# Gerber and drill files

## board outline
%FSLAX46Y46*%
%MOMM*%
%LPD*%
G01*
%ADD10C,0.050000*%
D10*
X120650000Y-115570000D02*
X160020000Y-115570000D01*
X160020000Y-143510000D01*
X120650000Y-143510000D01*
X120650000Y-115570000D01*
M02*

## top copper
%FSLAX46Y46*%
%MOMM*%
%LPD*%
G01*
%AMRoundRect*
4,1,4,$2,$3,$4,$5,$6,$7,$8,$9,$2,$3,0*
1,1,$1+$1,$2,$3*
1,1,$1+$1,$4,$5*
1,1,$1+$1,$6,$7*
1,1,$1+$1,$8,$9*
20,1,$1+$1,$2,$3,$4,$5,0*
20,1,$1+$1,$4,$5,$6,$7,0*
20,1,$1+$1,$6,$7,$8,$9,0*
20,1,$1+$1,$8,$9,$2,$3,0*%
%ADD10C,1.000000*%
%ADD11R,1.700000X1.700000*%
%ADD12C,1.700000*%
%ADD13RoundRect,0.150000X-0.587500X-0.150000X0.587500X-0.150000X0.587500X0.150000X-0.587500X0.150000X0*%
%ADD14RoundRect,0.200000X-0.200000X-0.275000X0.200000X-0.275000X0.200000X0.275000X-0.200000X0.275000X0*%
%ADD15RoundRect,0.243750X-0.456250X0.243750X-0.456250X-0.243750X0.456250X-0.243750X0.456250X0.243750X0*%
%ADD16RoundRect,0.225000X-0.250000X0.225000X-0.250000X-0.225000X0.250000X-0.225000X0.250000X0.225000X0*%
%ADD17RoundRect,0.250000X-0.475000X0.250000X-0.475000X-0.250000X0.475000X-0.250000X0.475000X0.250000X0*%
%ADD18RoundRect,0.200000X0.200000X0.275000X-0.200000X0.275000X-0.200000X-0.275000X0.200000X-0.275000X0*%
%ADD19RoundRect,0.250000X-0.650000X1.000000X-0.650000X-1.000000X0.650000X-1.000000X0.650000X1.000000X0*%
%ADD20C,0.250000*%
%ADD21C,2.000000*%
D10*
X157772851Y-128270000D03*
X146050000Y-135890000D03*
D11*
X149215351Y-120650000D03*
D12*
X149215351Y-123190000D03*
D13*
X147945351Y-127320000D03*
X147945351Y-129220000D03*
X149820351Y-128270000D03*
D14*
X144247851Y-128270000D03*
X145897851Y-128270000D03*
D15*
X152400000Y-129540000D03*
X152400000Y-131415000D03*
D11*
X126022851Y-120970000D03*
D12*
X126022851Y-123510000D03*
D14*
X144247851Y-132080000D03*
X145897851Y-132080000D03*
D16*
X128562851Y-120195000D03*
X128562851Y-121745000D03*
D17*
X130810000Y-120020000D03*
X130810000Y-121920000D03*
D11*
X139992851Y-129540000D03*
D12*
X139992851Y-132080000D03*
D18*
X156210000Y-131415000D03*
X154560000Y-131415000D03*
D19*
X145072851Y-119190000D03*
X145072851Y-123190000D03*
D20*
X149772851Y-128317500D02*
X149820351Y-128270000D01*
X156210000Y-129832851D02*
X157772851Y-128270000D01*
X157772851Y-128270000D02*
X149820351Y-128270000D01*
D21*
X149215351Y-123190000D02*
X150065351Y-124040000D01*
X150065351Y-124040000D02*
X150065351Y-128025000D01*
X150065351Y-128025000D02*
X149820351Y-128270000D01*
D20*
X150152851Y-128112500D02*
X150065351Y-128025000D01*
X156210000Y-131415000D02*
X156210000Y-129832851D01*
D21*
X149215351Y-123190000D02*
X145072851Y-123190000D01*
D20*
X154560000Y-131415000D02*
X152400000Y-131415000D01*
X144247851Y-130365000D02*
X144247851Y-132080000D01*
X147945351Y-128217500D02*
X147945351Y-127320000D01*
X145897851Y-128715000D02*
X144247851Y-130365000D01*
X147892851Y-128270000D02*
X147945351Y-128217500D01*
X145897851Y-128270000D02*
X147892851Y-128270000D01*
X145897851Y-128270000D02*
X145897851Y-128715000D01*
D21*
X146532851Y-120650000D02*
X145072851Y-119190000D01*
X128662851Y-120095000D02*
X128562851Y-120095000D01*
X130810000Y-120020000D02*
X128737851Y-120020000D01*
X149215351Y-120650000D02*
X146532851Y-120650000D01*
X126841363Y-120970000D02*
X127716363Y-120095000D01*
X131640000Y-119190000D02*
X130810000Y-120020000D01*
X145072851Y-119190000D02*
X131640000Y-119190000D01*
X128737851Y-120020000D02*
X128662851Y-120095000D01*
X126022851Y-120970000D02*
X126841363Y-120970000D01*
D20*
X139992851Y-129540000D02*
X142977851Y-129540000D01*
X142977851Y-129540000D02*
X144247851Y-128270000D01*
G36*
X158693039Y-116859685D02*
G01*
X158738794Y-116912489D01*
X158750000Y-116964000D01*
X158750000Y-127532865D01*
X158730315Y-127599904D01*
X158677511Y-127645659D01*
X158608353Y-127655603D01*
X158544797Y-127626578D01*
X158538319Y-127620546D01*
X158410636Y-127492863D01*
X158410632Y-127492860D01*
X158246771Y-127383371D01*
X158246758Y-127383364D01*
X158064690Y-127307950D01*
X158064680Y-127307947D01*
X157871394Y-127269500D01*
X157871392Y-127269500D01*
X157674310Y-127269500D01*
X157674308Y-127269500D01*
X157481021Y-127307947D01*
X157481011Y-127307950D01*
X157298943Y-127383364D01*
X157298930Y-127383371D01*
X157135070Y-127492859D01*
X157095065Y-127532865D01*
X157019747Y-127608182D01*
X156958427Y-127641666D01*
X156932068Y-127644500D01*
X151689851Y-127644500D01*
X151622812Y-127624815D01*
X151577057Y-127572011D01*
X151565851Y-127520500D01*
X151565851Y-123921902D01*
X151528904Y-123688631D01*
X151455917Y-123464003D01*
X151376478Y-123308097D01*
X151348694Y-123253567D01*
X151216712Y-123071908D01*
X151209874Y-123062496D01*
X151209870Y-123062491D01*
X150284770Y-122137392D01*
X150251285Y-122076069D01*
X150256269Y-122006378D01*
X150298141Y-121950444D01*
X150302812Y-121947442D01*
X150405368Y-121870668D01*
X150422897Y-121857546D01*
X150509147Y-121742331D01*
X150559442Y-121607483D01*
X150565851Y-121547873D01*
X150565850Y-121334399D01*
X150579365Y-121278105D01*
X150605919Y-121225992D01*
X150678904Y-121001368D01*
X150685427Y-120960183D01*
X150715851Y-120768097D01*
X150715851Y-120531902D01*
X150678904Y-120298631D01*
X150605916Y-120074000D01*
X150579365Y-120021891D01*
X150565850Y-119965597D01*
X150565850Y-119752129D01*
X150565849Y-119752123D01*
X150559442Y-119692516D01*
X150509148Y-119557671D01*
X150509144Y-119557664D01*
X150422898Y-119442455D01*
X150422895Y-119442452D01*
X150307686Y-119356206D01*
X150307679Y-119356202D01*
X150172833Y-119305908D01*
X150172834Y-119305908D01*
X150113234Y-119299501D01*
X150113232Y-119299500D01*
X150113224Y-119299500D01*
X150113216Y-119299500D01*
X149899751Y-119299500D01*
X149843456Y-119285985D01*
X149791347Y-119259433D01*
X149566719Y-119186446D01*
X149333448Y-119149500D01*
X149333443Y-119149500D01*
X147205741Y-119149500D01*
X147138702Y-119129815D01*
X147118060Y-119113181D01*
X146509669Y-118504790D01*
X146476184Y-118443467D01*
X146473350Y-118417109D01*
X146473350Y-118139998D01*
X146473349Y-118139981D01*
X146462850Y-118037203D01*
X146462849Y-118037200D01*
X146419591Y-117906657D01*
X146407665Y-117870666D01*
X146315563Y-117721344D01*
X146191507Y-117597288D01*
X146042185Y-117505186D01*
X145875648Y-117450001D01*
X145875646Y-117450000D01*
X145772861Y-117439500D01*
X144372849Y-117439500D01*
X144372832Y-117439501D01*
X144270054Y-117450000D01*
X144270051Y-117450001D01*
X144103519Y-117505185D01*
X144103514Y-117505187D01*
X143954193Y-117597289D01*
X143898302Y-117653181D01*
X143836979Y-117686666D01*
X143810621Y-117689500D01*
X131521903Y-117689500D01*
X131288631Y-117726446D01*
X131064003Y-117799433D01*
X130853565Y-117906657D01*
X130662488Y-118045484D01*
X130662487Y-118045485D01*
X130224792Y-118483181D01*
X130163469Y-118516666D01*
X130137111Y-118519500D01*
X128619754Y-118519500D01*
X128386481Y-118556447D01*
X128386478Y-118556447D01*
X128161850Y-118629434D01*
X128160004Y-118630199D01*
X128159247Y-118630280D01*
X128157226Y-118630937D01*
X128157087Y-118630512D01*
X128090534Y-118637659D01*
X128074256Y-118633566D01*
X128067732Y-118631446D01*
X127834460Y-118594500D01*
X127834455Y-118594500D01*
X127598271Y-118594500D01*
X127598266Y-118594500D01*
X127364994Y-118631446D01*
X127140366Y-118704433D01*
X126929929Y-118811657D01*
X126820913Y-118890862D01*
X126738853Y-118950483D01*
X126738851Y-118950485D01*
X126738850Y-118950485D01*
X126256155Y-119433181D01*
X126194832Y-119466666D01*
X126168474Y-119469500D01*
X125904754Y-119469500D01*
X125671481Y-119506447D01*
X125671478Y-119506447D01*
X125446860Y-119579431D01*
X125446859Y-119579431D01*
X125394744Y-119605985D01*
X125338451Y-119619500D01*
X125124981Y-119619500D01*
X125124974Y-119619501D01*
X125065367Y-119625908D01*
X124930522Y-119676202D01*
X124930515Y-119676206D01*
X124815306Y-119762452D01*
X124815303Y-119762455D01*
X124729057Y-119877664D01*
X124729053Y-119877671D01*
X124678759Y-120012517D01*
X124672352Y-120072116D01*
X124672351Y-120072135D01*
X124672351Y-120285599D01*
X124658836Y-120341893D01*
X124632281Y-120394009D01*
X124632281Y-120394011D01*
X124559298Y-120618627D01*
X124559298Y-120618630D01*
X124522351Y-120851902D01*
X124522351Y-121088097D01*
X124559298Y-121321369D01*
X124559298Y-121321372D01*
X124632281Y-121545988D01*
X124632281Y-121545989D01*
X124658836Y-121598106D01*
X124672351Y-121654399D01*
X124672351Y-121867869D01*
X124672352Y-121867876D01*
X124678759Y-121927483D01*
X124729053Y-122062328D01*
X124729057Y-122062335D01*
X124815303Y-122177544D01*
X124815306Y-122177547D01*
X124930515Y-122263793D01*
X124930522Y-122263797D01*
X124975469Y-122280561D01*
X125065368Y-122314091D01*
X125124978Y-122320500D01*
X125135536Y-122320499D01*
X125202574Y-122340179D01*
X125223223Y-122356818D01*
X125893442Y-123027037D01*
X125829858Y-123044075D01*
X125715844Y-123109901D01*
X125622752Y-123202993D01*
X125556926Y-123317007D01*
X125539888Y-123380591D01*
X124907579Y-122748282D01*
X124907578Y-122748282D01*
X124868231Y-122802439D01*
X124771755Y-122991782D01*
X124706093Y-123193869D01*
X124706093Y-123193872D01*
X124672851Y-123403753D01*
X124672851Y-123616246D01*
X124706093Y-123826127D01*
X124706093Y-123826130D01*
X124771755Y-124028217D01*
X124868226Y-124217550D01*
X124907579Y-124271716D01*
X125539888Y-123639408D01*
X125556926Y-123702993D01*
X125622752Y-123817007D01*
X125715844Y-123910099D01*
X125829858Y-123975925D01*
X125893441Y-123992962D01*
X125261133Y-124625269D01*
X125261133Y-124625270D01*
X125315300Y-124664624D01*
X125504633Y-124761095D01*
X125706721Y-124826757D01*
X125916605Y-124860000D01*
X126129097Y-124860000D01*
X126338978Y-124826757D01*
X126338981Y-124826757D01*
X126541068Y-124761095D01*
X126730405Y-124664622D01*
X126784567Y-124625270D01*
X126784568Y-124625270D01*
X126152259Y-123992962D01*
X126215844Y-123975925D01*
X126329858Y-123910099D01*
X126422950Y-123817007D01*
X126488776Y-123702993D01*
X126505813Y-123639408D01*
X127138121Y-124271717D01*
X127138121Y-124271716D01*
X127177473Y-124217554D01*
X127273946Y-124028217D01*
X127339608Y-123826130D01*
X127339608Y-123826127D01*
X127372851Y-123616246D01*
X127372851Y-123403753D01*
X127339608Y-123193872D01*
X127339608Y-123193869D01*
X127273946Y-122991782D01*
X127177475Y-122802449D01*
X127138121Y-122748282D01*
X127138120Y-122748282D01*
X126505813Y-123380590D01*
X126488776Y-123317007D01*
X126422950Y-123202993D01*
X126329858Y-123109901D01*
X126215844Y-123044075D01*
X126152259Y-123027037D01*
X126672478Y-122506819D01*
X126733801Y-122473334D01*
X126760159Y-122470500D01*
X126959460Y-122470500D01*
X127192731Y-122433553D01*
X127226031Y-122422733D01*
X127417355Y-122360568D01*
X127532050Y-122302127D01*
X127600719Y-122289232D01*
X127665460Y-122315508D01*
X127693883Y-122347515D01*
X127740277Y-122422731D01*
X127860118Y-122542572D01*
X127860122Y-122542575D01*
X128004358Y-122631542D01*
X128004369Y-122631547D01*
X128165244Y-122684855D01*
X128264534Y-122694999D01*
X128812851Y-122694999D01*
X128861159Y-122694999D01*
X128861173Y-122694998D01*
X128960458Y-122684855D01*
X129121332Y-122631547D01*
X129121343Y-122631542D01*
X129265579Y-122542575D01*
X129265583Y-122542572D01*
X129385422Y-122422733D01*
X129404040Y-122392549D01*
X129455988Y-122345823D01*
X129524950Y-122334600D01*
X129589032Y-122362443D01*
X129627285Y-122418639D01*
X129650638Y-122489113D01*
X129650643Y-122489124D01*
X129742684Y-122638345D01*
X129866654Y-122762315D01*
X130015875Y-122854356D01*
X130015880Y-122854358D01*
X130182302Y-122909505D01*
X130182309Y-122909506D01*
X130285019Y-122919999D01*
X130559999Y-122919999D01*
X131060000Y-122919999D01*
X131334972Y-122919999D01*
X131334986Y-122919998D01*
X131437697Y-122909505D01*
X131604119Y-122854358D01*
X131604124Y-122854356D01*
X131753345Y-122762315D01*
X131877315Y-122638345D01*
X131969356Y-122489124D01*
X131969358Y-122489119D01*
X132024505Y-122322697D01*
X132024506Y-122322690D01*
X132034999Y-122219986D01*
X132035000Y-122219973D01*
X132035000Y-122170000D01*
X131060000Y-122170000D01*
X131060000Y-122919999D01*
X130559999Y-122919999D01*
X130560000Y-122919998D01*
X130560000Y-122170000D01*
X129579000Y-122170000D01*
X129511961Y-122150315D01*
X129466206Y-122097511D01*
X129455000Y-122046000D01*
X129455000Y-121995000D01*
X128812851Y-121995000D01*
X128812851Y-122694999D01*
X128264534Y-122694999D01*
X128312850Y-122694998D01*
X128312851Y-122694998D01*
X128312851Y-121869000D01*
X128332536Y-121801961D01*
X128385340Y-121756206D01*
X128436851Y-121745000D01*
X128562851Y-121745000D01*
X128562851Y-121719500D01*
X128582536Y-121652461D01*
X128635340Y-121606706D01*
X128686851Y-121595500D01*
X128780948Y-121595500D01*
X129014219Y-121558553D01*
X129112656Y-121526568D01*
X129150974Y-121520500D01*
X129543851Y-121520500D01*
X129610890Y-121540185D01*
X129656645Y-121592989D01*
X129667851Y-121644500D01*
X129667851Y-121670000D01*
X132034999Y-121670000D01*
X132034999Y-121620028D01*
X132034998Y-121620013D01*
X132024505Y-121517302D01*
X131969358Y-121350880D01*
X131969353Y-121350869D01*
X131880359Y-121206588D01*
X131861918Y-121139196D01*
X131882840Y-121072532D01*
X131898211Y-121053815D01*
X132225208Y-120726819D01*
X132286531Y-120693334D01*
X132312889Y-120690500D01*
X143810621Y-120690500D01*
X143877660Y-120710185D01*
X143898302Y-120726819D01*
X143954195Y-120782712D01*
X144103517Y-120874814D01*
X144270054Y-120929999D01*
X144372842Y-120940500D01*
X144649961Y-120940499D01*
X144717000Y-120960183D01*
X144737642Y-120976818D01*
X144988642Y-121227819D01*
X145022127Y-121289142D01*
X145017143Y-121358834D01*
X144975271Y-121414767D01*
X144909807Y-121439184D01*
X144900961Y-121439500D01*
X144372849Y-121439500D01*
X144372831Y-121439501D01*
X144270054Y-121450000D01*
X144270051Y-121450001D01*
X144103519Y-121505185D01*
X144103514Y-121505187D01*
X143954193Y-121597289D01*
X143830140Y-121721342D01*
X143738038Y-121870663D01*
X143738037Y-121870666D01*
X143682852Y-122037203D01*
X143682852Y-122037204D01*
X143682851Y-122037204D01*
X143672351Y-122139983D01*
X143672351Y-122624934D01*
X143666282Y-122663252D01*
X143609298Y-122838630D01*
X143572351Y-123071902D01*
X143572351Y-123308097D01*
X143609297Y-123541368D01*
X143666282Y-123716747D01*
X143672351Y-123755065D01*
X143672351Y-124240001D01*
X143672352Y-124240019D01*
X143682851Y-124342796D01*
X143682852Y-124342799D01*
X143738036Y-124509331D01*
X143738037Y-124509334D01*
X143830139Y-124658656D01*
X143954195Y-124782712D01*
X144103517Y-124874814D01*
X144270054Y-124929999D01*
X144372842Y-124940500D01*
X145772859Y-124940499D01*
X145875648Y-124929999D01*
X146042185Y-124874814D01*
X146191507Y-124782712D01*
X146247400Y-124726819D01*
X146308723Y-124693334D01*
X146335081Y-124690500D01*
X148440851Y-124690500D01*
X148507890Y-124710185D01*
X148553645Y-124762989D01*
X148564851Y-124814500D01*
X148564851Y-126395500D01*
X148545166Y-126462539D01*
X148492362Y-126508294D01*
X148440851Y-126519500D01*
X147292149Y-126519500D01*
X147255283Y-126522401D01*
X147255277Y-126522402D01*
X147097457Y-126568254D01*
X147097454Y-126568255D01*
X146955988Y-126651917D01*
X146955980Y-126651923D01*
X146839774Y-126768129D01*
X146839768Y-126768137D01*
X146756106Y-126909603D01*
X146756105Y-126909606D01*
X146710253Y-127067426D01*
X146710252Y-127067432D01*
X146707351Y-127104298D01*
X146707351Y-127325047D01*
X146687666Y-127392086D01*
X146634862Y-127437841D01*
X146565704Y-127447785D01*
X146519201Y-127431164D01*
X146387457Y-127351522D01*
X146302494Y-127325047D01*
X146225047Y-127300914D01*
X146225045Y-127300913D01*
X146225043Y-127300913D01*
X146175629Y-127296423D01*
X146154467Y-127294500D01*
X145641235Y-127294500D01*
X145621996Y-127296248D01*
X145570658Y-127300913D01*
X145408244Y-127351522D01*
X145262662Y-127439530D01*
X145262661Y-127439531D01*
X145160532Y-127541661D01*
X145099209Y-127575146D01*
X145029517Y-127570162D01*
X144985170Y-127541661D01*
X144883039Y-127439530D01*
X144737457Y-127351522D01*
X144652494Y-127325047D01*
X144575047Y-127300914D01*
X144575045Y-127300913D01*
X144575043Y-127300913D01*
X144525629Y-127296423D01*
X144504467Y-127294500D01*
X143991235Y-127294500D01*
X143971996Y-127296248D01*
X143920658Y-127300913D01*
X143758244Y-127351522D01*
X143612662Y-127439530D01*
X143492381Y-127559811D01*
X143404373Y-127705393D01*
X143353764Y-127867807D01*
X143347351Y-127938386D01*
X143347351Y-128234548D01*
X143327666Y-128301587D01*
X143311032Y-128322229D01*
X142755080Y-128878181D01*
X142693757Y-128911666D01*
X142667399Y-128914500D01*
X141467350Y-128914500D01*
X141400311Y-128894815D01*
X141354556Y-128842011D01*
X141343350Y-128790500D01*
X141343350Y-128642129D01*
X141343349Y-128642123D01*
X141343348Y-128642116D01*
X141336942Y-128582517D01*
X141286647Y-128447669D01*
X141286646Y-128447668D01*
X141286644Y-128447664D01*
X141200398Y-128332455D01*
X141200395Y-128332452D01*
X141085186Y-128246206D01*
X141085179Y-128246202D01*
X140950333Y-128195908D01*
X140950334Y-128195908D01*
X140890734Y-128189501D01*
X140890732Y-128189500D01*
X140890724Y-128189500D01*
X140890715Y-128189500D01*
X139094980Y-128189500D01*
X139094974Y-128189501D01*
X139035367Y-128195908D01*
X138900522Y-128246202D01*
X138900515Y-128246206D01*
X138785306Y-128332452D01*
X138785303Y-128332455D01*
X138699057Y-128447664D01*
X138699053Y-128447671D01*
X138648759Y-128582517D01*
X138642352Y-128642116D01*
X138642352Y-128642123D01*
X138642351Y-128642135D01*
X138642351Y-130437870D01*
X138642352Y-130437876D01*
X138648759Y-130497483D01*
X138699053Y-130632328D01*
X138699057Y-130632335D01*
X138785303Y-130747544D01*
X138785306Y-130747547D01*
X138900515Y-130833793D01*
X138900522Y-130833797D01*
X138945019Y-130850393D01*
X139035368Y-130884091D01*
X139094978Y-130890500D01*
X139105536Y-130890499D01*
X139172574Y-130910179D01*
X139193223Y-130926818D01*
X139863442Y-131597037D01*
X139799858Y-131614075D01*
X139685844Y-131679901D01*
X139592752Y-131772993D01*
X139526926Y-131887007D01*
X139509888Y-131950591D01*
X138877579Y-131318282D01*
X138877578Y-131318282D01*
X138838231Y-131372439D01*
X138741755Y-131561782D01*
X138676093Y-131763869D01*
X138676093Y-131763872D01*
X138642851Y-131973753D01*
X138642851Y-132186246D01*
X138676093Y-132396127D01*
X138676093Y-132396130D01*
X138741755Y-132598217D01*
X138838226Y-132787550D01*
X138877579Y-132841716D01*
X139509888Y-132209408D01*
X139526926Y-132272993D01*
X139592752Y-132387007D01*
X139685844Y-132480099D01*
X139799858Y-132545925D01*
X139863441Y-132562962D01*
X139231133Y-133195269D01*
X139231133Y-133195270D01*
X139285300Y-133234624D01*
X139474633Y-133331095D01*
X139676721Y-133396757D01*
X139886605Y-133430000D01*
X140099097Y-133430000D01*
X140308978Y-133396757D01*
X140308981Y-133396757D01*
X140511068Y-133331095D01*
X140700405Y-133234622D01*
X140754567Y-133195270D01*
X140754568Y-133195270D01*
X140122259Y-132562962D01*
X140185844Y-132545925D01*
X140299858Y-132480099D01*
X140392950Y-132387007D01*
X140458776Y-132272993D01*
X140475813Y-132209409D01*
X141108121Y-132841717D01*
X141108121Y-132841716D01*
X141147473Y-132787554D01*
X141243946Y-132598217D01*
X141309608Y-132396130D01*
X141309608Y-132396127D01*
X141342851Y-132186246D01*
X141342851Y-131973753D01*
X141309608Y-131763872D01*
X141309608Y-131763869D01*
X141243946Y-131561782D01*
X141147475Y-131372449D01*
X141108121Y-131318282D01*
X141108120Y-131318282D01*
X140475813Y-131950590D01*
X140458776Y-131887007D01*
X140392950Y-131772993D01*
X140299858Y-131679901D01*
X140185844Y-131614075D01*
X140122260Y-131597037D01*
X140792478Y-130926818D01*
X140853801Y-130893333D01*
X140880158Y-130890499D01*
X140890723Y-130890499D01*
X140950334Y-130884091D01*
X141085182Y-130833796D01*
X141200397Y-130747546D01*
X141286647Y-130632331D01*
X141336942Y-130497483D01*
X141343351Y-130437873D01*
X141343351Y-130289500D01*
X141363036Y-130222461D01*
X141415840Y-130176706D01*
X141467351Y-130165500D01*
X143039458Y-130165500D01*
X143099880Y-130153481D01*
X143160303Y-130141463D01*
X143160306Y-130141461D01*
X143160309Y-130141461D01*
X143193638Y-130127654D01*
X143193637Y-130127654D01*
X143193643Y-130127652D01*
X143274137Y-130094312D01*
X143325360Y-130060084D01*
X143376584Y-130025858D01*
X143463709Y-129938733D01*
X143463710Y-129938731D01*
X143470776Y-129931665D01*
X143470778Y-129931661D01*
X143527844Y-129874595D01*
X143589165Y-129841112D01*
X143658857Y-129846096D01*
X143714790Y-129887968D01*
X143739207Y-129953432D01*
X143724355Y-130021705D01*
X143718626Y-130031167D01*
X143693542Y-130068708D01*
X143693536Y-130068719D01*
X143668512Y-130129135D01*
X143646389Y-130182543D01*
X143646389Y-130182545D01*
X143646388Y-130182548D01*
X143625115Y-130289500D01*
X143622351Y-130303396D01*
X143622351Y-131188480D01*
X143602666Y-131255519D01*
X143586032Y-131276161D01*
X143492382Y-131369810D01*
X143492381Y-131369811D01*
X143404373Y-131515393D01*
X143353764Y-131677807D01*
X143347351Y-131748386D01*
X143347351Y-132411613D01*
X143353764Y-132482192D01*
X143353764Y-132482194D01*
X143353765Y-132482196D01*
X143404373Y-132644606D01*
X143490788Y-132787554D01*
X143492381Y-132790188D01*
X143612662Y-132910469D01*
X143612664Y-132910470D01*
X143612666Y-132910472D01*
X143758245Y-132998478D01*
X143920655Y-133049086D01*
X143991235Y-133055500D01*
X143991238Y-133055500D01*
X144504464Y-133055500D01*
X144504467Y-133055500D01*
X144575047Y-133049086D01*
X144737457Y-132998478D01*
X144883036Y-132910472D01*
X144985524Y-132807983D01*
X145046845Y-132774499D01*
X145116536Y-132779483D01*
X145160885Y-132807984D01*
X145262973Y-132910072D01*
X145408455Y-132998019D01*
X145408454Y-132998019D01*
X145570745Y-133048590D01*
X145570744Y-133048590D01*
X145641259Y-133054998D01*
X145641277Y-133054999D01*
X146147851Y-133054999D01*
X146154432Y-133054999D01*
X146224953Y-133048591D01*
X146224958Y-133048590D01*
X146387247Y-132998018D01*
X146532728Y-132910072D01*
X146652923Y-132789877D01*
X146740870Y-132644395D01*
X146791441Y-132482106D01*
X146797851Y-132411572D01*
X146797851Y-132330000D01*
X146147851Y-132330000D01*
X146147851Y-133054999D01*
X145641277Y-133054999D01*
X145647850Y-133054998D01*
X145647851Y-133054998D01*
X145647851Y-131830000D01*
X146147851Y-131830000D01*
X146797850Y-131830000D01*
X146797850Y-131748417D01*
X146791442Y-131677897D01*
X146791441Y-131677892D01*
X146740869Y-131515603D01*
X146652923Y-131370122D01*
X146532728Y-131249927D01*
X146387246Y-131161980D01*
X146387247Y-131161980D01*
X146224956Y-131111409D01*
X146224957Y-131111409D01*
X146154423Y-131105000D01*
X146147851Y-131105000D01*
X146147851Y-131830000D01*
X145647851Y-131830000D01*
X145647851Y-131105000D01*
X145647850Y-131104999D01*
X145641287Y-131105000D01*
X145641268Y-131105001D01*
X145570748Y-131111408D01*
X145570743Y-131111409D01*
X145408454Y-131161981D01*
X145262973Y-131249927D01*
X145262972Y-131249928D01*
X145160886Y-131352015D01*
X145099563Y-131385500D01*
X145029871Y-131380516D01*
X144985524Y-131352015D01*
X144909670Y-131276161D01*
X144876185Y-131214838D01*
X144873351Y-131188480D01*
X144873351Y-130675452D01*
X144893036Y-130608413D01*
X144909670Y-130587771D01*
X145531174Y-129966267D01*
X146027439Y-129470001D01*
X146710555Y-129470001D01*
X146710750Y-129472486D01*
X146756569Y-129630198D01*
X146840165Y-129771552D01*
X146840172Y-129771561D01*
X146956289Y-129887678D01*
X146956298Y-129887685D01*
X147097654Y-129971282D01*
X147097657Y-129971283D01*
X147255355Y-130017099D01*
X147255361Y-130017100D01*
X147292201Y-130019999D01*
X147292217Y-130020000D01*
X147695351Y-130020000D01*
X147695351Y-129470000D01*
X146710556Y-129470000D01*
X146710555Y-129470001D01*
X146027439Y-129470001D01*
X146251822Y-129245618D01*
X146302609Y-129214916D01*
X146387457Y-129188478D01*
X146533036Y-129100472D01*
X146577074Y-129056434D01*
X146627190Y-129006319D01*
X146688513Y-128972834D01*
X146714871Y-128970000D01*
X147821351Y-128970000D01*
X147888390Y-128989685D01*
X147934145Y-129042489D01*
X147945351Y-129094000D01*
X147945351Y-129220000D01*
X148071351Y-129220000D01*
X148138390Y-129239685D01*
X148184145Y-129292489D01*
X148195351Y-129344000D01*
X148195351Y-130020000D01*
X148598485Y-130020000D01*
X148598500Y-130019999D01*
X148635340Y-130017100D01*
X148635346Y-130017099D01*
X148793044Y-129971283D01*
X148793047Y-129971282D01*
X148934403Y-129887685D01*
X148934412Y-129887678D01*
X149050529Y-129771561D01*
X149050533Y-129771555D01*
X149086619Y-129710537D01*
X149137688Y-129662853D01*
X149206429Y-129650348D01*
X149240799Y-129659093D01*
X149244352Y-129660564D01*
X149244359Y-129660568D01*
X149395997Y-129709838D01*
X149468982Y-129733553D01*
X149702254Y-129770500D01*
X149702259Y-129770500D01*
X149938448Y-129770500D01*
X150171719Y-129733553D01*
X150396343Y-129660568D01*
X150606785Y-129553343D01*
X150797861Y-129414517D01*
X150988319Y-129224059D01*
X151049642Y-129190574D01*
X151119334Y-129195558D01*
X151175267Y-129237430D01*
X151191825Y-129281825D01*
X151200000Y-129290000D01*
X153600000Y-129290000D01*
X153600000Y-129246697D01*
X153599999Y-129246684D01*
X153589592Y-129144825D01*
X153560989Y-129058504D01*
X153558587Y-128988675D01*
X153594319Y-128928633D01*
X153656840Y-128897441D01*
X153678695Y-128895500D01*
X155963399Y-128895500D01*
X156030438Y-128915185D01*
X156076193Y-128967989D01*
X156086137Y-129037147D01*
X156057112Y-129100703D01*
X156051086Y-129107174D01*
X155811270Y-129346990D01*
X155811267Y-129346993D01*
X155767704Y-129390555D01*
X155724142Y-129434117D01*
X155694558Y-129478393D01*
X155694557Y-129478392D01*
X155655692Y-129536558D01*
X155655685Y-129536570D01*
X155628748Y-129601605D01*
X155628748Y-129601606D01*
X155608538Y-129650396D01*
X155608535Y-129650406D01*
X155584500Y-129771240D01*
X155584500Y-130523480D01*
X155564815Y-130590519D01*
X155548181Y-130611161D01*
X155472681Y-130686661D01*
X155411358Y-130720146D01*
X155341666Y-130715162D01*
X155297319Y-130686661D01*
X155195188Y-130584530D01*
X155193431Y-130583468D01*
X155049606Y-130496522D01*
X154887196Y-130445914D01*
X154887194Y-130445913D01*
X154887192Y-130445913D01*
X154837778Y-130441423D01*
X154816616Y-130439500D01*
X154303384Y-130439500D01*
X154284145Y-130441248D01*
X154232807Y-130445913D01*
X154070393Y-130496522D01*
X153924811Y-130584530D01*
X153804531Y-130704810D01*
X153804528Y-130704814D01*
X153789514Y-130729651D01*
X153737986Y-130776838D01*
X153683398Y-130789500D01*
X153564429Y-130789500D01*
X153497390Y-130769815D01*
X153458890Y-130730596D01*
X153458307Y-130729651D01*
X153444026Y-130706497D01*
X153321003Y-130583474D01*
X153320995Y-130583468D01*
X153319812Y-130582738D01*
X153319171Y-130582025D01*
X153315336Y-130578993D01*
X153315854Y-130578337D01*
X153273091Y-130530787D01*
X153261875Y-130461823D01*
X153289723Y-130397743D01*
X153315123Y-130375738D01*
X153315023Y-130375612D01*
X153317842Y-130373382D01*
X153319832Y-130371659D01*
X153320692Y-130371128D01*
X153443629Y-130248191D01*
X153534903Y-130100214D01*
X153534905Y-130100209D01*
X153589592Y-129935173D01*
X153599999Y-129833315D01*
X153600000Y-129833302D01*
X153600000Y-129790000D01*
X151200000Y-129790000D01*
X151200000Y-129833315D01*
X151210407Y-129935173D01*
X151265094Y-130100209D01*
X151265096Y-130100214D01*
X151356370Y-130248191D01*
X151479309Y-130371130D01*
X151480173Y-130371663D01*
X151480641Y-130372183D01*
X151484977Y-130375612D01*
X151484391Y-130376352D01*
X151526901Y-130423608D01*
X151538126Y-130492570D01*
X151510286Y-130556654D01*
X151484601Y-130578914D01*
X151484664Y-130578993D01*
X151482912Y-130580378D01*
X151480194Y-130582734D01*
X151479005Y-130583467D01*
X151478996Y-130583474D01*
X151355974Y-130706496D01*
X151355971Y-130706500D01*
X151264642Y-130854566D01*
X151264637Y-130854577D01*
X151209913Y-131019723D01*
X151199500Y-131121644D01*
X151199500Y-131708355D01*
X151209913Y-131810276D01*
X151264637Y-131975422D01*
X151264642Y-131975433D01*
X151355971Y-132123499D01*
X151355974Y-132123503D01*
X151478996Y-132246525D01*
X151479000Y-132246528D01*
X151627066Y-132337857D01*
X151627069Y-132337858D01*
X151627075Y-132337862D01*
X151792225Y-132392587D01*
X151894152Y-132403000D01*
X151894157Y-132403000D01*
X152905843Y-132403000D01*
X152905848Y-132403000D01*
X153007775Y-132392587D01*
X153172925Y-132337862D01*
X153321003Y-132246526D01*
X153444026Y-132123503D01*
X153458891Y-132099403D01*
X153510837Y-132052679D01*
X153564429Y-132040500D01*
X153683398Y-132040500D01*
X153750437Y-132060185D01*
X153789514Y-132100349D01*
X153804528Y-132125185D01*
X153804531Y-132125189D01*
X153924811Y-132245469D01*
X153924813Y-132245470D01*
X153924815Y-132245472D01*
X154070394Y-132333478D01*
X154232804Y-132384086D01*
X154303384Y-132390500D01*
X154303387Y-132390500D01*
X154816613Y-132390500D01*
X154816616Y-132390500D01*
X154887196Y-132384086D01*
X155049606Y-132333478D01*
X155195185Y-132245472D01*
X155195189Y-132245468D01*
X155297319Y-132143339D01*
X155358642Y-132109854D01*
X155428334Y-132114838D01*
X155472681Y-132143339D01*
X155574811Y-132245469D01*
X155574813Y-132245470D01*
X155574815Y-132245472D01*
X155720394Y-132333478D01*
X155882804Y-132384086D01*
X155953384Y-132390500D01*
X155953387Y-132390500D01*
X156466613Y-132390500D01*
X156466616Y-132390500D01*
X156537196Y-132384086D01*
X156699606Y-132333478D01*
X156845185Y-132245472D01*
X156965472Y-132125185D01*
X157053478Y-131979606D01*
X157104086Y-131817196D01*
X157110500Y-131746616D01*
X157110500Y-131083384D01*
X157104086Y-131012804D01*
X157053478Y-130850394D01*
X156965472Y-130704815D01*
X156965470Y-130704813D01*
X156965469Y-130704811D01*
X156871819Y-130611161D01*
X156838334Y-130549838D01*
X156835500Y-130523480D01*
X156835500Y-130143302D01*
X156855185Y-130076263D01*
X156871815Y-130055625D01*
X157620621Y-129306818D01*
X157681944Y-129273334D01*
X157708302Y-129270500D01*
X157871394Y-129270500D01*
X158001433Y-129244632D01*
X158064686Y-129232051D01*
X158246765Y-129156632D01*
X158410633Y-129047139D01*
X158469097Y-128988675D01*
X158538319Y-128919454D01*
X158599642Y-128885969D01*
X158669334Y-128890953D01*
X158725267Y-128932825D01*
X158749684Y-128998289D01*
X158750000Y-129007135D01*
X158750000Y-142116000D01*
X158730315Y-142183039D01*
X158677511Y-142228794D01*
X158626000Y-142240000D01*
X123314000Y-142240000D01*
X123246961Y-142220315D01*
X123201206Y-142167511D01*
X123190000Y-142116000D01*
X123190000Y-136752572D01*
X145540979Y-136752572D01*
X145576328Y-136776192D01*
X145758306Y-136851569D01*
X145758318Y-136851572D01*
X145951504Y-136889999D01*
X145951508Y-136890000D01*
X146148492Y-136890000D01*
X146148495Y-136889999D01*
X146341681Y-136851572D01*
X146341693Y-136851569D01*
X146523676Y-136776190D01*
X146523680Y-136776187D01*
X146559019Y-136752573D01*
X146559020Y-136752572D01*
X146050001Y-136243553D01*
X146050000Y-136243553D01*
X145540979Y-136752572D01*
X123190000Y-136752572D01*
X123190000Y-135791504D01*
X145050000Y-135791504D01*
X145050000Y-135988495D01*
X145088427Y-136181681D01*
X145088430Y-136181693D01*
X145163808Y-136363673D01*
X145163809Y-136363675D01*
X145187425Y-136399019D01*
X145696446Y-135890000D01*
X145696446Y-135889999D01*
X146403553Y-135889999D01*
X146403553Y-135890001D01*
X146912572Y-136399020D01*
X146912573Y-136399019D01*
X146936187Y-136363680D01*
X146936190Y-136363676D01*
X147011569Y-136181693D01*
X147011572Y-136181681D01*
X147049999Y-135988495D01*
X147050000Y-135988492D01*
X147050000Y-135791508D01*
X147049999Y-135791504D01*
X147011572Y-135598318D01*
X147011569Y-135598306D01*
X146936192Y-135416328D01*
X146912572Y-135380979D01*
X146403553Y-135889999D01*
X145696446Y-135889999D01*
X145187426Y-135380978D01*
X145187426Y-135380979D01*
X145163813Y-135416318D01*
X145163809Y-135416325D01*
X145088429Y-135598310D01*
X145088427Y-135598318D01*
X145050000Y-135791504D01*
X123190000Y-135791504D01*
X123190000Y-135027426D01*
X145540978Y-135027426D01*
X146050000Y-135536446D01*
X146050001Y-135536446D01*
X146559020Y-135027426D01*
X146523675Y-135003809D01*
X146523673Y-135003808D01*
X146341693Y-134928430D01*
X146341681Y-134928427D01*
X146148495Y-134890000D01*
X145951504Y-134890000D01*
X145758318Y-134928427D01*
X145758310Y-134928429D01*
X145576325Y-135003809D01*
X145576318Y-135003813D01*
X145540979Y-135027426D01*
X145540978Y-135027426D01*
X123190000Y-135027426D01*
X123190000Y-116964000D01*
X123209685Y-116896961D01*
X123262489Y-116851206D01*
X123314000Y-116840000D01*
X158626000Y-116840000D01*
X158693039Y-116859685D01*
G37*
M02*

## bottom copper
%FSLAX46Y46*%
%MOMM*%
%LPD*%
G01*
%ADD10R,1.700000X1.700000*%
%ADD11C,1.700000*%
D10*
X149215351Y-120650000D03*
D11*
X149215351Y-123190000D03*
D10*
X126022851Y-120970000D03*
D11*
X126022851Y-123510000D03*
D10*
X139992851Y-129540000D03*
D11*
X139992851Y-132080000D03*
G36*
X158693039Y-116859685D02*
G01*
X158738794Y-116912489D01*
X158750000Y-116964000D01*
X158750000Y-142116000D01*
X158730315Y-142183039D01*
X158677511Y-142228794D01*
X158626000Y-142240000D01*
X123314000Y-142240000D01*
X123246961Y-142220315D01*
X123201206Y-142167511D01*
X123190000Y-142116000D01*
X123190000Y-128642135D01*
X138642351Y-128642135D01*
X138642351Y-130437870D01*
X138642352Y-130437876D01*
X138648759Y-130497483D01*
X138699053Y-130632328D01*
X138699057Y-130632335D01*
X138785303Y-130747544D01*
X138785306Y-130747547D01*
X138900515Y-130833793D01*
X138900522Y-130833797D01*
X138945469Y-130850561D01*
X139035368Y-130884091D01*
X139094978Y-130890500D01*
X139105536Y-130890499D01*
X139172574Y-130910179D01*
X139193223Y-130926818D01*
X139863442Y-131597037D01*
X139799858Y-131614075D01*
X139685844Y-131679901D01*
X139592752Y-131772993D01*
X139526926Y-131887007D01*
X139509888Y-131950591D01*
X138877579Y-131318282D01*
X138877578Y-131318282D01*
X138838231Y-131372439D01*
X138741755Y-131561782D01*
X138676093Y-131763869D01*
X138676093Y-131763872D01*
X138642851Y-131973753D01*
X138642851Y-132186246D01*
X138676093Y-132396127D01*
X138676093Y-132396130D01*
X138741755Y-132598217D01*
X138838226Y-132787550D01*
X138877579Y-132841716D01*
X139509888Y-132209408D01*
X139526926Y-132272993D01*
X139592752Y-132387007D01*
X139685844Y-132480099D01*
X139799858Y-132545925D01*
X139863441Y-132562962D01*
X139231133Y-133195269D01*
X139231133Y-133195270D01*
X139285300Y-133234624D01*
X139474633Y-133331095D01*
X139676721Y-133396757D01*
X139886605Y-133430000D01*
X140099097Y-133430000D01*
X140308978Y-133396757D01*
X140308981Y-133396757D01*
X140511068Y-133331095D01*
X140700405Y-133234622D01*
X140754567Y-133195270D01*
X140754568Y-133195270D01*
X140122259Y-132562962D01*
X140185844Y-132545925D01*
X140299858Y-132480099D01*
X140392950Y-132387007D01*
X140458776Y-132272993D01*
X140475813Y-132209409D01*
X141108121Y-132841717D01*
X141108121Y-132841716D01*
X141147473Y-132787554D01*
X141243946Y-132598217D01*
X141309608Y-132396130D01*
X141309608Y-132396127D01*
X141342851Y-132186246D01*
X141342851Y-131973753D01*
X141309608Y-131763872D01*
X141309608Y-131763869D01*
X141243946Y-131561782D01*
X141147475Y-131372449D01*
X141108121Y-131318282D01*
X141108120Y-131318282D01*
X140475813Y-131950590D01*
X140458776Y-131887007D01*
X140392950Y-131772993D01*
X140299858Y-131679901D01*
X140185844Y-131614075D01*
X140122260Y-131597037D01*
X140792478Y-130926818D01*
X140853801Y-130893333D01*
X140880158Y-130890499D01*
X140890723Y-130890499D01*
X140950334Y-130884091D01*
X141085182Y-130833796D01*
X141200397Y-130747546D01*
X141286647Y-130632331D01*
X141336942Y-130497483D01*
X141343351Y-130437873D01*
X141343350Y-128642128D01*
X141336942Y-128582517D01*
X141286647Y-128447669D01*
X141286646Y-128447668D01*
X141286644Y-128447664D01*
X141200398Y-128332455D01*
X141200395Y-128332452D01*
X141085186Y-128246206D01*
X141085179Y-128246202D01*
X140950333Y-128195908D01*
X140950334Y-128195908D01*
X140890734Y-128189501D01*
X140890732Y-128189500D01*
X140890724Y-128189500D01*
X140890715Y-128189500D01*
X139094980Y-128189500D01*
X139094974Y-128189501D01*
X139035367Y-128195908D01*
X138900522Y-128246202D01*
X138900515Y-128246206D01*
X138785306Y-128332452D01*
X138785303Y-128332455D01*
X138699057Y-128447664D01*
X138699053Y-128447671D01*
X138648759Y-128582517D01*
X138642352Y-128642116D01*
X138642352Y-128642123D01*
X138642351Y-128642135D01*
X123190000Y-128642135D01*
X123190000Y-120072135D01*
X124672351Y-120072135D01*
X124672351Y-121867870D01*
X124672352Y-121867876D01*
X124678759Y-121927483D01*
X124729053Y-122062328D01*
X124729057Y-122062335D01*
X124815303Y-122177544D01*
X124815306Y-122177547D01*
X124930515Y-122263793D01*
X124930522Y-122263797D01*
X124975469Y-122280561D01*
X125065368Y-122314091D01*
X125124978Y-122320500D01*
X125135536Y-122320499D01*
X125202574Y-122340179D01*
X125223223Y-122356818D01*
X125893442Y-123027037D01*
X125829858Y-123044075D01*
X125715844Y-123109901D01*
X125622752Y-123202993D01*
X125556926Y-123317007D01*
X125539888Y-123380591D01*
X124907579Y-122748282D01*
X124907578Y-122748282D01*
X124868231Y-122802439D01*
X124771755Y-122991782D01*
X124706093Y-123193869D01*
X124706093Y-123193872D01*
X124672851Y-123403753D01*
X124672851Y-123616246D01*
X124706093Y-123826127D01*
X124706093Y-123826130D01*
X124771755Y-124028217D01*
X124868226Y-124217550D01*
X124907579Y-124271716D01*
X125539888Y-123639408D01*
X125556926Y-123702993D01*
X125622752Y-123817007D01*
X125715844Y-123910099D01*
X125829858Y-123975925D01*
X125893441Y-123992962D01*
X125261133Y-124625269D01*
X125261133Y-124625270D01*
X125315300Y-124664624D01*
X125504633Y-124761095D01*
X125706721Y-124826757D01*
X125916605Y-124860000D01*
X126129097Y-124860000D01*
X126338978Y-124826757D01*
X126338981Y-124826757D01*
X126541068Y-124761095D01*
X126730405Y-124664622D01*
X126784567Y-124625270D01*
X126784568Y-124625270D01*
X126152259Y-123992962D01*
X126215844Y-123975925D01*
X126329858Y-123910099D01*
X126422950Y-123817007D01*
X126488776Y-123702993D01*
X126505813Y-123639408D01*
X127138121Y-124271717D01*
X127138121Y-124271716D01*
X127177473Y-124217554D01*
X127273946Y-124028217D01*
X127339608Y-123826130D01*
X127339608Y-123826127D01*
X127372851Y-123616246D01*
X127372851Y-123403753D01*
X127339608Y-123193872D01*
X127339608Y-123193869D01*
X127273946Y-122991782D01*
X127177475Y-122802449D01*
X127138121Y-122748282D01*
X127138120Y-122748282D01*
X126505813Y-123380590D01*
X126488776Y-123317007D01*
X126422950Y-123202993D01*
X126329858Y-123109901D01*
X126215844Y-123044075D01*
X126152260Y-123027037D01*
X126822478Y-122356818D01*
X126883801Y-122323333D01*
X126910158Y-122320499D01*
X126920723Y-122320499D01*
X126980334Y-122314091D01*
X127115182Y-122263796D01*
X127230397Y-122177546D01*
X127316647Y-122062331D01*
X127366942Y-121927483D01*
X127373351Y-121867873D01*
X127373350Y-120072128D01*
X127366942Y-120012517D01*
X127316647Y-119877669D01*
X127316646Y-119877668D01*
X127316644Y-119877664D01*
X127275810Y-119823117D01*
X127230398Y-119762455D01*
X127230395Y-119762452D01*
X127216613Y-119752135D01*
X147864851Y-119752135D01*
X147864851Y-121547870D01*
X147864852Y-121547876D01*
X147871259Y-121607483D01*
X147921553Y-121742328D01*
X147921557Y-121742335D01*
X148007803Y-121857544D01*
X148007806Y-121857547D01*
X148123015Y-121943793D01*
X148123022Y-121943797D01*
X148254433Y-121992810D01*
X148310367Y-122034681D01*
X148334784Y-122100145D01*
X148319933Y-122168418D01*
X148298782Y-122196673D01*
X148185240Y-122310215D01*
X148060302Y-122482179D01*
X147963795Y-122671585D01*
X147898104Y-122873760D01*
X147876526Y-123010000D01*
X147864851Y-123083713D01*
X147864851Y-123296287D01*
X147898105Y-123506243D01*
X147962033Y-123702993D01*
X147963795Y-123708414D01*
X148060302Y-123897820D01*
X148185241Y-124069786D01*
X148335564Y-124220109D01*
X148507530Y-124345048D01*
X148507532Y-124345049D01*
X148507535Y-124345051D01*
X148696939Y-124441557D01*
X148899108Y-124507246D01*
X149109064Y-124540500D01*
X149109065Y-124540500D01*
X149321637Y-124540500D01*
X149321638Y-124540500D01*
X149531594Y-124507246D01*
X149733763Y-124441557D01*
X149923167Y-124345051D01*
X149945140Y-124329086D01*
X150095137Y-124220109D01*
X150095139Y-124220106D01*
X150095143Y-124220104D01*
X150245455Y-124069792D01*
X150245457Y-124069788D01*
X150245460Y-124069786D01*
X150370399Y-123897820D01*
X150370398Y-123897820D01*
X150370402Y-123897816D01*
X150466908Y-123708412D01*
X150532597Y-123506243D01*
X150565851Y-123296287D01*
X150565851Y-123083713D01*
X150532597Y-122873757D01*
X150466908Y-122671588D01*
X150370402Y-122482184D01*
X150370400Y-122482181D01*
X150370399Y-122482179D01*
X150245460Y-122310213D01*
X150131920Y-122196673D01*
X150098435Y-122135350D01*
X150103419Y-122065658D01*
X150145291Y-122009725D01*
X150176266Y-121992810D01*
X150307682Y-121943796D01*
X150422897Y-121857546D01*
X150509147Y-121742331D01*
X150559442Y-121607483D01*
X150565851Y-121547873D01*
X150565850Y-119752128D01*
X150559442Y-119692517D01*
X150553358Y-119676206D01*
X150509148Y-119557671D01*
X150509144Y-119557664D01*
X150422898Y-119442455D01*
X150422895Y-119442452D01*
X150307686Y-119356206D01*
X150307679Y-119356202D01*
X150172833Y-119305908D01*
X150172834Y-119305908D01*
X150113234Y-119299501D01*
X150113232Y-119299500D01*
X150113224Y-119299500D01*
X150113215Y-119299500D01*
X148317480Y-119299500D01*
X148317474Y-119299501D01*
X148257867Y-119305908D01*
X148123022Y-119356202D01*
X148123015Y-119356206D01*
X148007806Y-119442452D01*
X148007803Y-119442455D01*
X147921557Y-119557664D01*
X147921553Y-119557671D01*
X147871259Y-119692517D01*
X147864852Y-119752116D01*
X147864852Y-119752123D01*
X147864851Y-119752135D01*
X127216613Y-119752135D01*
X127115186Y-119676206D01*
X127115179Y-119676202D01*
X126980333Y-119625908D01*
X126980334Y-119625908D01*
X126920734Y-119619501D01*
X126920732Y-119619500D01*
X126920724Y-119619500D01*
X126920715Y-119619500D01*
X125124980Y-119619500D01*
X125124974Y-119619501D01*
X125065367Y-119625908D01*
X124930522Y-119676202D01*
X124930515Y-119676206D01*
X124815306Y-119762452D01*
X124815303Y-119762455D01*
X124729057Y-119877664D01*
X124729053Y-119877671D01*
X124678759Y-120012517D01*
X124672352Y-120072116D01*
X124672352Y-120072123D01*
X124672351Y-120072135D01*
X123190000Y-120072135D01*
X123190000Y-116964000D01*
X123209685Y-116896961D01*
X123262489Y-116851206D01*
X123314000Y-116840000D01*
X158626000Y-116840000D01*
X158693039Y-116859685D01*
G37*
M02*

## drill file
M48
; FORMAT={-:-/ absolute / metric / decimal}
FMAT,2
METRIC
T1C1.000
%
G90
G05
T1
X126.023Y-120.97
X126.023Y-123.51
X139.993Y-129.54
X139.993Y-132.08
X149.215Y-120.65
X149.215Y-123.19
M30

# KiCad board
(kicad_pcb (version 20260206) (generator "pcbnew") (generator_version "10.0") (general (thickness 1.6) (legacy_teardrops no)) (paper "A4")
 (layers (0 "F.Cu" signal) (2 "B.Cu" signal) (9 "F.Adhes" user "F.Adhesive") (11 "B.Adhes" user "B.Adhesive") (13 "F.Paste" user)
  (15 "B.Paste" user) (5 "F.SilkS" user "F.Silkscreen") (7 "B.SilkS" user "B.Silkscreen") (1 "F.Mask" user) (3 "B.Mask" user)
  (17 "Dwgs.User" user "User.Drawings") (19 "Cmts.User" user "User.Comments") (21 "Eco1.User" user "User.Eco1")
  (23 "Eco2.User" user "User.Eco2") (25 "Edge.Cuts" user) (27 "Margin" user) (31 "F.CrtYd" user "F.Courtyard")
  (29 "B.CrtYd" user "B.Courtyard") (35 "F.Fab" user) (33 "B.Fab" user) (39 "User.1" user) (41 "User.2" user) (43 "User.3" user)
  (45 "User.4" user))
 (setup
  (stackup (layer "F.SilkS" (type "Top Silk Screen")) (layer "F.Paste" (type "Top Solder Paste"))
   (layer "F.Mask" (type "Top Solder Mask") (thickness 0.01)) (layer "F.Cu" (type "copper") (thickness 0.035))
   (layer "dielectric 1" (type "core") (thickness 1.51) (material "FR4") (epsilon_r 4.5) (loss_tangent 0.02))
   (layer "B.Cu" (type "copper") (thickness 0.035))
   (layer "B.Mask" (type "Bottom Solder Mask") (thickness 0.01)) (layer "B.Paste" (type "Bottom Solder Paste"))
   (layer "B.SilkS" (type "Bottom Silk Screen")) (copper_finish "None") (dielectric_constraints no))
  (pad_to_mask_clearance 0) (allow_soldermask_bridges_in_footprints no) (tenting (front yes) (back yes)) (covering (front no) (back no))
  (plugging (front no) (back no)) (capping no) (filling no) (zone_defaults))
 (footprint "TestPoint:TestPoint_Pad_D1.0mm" (layer "F.Cu") (at 157.772851 128.27)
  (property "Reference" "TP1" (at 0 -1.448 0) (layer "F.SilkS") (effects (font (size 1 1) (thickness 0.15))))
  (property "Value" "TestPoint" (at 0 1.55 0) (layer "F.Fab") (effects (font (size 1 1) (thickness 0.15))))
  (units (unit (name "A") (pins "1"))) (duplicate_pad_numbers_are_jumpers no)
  (pad "1" smd circle (at 0 0) (size 1 1) (layers "F.Cu" "F.Mask") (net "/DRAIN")))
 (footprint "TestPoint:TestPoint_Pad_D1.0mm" (layer "F.Cu") (at 146.05 135.89)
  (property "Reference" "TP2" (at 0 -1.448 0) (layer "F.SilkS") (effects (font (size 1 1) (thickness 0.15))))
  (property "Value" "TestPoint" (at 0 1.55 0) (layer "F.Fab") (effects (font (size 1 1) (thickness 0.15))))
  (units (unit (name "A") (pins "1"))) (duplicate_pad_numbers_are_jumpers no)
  (pad "1" smd circle (at 0 0) (size 1 1) (layers "F.Cu" "F.Mask") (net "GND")))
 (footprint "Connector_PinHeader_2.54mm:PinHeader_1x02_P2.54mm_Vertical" (layer "F.Cu") (at 149.215351 120.65)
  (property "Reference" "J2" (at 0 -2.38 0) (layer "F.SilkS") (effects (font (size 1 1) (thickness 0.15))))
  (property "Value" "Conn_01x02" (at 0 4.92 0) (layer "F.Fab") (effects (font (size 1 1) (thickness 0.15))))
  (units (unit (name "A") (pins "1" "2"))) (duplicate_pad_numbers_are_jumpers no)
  (pad "1" thru_hole rect (at 0 0) (size 1.7 1.7) (drill 1) (layers "*.Cu" "*.Mask") (remove_unused_layers no) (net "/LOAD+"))
  (pad "2" thru_hole circle (at 0 2.54) (size 1.7 1.7) (drill 1) (layers "*.Cu" "*.Mask") (remove_unused_layers no) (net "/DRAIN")))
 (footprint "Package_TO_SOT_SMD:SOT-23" (layer "F.Cu") (at 148.882851 128.27)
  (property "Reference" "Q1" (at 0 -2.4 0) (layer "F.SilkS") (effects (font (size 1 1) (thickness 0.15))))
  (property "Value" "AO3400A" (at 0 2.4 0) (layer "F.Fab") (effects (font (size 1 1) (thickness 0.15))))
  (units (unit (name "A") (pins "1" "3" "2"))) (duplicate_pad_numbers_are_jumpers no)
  (pad "1" smd roundrect (at -0.9375 -0.95) (size 1.475 0.6) (layers "F.Cu" "F.Mask" "F.Paste") (roundrect_rratio 0.25) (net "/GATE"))
  (pad "2" smd roundrect (at -0.9375 0.95) (size 1.475 0.6) (layers "F.Cu" "F.Mask" "F.Paste") (roundrect_rratio 0.25) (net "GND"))
  (pad "3" smd roundrect (at 0.9375 0) (size 1.475 0.6) (layers "F.Cu" "F.Mask" "F.Paste") (roundrect_rratio 0.25) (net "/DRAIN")))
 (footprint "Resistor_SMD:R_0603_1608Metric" (layer "F.Cu") (at 145.072851 128.27)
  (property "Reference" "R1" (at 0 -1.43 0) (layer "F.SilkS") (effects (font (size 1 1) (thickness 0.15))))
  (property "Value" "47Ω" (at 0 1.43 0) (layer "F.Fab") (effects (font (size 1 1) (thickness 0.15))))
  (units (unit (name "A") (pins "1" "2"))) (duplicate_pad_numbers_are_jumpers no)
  (pad "1" smd roundrect (at -0.825 0) (size 0.8 0.95) (layers "F.Cu" "F.Mask" "F.Paste") (roundrect_rratio 0.25) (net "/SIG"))
  (pad "2" smd roundrect (at 0.825 0) (size 0.8 0.95) (layers "F.Cu" "F.Mask" "F.Paste") (roundrect_rratio 0.25) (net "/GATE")))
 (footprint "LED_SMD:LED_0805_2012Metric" (layer "F.Cu") (at 152.4 130.4775 -90)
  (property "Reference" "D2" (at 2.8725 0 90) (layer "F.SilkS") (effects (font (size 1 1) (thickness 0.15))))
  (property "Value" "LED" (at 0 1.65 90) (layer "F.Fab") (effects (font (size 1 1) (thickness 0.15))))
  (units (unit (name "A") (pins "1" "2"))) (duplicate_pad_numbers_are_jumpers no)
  (pad "1" smd roundrect (at -0.9375 0 270) (size 0.975 1.4) (layers "F.Cu" "F.Mask" "F.Paste") (roundrect_rratio 0.25) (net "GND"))
  (pad "2" smd roundrect (at 0.9375 0 270) (size 0.975 1.4) (layers "F.Cu" "F.Mask" "F.Paste") (roundrect_rratio 0.25) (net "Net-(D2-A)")))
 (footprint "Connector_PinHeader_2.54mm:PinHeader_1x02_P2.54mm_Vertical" (layer "F.Cu") (at 126.022851 120.97)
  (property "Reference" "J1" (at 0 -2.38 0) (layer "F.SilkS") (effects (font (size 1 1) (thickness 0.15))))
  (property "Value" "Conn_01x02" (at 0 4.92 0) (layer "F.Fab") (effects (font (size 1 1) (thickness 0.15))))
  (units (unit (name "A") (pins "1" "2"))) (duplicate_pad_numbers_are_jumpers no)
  (pad "1" thru_hole rect (at 0 0) (size 1.7 1.7) (drill 1) (layers "*.Cu" "*.Mask") (remove_unused_layers no) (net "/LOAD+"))
  (pad "2" thru_hole circle (at 0 2.54) (size 1.7 1.7) (drill 1) (layers "*.Cu" "*.Mask") (remove_unused_layers no) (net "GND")))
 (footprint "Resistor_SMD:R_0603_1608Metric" (layer "F.Cu") (at 145.072851 132.08)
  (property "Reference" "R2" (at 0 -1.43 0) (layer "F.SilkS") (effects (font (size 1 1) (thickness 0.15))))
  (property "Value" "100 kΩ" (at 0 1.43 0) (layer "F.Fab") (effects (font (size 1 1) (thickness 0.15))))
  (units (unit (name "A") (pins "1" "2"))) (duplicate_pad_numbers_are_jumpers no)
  (pad "1" smd roundrect (at -0.825 0) (size 0.8 0.95) (layers "F.Cu" "F.Mask" "F.Paste") (roundrect_rratio 0.25) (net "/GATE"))
  (pad "2" smd roundrect (at 0.825 0) (size 0.8 0.95) (layers "F.Cu" "F.Mask" "F.Paste") (roundrect_rratio 0.25) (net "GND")))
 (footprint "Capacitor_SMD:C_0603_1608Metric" (layer "F.Cu") (at 128.562851 120.97 -90)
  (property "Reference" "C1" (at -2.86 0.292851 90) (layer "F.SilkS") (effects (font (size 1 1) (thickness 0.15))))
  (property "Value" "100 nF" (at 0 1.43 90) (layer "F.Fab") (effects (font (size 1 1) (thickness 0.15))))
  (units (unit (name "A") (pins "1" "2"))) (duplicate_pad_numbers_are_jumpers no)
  (pad "1" smd roundrect (at -0.775 0 270) (size 0.9 0.95) (layers "F.Cu" "F.Mask" "F.Paste") (roundrect_rratio 0.25) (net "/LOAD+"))
  (pad "2" smd roundrect (at 0.775 0 270) (size 0.9 0.95) (layers "F.Cu" "F.Mask" "F.Paste") (roundrect_rratio 0.25) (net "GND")))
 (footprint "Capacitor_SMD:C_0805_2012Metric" (layer "F.Cu") (at 130.81 120.97 -90)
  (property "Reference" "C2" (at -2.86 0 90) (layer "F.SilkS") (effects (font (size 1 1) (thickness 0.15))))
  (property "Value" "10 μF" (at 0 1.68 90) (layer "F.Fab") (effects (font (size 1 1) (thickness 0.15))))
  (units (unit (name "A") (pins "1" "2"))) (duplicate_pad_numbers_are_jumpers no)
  (pad "1" smd roundrect (at -0.95 0 270) (size 1 1.45) (layers "F.Cu" "F.Mask" "F.Paste") (roundrect_rratio 0.25) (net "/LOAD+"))
  (pad "2" smd roundrect (at 0.95 0 270) (size 1 1.45) (layers "F.Cu" "F.Mask" "F.Paste") (roundrect_rratio 0.25) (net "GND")))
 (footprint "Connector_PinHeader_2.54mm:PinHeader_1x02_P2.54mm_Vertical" (layer "F.Cu") (at 139.992851 129.54)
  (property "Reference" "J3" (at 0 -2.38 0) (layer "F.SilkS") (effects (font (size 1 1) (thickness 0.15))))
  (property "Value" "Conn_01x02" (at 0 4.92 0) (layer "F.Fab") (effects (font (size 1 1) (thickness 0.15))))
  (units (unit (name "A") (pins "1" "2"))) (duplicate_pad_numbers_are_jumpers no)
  (pad "1" thru_hole rect (at 0 0) (size 1.7 1.7) (drill 1) (layers "*.Cu" "*.Mask") (remove_unused_layers no) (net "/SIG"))
  (pad "2" thru_hole circle (at 0 2.54) (size 1.7 1.7) (drill 1) (layers "*.Cu" "*.Mask") (remove_unused_layers no) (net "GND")))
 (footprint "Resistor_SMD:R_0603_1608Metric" (layer "F.Cu") (at 155.385 131.415 180)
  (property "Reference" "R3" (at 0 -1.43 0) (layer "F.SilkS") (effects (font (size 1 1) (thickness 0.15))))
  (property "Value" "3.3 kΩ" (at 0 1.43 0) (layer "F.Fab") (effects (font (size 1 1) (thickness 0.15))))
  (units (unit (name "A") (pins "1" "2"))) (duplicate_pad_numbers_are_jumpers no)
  (pad "1" smd roundrect (at -0.825 0 180) (size 0.8 0.95) (layers "F.Cu" "F.Mask" "F.Paste") (roundrect_rratio 0.25) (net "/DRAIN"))
  (pad "2" smd roundrect (at 0.825 0 180) (size 0.8 0.95) (layers "F.Cu" "F.Mask" "F.Paste") (roundrect_rratio 0.25) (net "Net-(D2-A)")))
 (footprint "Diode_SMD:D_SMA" (layer "F.Cu") (at 145.072851 121.19 -90)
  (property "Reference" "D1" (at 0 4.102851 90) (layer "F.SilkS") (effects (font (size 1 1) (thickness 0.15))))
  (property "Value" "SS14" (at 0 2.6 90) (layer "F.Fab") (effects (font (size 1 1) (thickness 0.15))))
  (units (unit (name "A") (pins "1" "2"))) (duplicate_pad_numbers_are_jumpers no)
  (pad "1" smd roundrect (at -2 0 270) (size 2.5 1.8) (layers "F.Cu" "F.Mask" "F.Paste") (roundrect_rratio 0.1388888889) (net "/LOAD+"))
  (pad "2" smd roundrect (at 2 0 270) (size 2.5 1.8) (layers "F.Cu" "F.Mask" "F.Paste") (roundrect_rratio 0.1388888889) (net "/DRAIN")))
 (gr_rect (start 120.65 115.57) (end 160.02 143.51) (stroke (width 0.05) (type default)) (fill no) (layer "Edge.Cuts"))
 (segment (start 149.772851 128.3175) (end 149.820351 128.27) (width 0.25) (layer "F.Cu") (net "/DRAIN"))
 (segment (start 156.21 129.832851) (end 157.772851 128.27) (width 0.25) (layer "F.Cu") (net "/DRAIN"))
 (segment (start 157.772851 128.27) (end 149.820351 128.27) (width 0.25) (layer "F.Cu") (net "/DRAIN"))
 (segment (start 149.215351 123.19) (end 150.065351 124.04) (width 2) (layer "F.Cu") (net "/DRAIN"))
 (segment (start 150.065351 124.04) (end 150.065351 128.025) (width 2) (layer "F.Cu") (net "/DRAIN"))
 (segment (start 150.065351 128.025) (end 149.820351 128.27) (width 2) (layer "F.Cu") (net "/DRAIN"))
 (segment (start 150.152851 128.1125) (end 150.065351 128.025) (width 0.25) (layer "F.Cu") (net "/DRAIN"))
 (segment (start 156.21 131.415) (end 156.21 129.832851) (width 0.25) (layer "F.Cu") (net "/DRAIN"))
 (segment (start 149.215351 123.19) (end 145.072851 123.19) (width 2) (layer "F.Cu") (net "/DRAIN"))
 (segment (start 154.56 131.415) (end 152.4 131.415) (width 0.25) (layer "F.Cu") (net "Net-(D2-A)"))
 (segment (start 144.247851 130.365) (end 144.247851 132.08) (width 0.25) (layer "F.Cu") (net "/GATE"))
 (segment (start 147.945351 128.2175) (end 147.945351 127.32) (width 0.25) (layer "F.Cu") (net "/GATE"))
 (segment (start 145.897851 128.715) (end 144.247851 130.365) (width 0.25) (layer "F.Cu") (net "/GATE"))
 (segment (start 147.892851 128.27) (end 147.945351 128.2175) (width 0.25) (layer "F.Cu") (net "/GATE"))
 (segment (start 145.897851 128.27) (end 147.892851 128.27) (width 0.25) (layer "F.Cu") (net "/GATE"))
 (segment (start 145.897851 128.27) (end 145.897851 128.715) (width 0.25) (layer "F.Cu") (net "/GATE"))
 (segment (start 146.532851 120.65) (end 145.072851 119.19) (width 2) (layer "F.Cu") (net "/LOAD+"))
 (segment (start 128.662851 120.095) (end 128.562851 120.095) (width 2) (layer "F.Cu") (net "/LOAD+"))
 (segment (start 130.81 120.02) (end 128.737851 120.02) (width 2) (layer "F.Cu") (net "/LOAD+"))
 (segment (start 149.215351 120.65) (end 146.532851 120.65) (width 2) (layer "F.Cu") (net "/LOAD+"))
 (segment (start 126.841363 120.97) (end 127.716363 120.095) (width 2) (layer "F.Cu") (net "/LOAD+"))
 (segment (start 131.64 119.19) (end 130.81 120.02) (width 2) (layer "F.Cu") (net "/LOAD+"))
 (segment (start 145.072851 119.19) (end 131.64 119.19) (width 2) (layer "F.Cu") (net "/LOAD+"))
 (segment (start 128.737851 120.02) (end 128.662851 120.095) (width 2) (layer "F.Cu") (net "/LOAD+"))
 (segment (start 126.022851 120.97) (end 126.841363 120.97) (width 2) (layer "F.Cu") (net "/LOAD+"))
 (segment (start 139.992851 129.54) (end 142.977851 129.54) (width 0.25) (layer "F.Cu") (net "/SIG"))
 (segment (start 142.977851 129.54) (end 144.247851 128.27) (width 0.25) (layer "F.Cu") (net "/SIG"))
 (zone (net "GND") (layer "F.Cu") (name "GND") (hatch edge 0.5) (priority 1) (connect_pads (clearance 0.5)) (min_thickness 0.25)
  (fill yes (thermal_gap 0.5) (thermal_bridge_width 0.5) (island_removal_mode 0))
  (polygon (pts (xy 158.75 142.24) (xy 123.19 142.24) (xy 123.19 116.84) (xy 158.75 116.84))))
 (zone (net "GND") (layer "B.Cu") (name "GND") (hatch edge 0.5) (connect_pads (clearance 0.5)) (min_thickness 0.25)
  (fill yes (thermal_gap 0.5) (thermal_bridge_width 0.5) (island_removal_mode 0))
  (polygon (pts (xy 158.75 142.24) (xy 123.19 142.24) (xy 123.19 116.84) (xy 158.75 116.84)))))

